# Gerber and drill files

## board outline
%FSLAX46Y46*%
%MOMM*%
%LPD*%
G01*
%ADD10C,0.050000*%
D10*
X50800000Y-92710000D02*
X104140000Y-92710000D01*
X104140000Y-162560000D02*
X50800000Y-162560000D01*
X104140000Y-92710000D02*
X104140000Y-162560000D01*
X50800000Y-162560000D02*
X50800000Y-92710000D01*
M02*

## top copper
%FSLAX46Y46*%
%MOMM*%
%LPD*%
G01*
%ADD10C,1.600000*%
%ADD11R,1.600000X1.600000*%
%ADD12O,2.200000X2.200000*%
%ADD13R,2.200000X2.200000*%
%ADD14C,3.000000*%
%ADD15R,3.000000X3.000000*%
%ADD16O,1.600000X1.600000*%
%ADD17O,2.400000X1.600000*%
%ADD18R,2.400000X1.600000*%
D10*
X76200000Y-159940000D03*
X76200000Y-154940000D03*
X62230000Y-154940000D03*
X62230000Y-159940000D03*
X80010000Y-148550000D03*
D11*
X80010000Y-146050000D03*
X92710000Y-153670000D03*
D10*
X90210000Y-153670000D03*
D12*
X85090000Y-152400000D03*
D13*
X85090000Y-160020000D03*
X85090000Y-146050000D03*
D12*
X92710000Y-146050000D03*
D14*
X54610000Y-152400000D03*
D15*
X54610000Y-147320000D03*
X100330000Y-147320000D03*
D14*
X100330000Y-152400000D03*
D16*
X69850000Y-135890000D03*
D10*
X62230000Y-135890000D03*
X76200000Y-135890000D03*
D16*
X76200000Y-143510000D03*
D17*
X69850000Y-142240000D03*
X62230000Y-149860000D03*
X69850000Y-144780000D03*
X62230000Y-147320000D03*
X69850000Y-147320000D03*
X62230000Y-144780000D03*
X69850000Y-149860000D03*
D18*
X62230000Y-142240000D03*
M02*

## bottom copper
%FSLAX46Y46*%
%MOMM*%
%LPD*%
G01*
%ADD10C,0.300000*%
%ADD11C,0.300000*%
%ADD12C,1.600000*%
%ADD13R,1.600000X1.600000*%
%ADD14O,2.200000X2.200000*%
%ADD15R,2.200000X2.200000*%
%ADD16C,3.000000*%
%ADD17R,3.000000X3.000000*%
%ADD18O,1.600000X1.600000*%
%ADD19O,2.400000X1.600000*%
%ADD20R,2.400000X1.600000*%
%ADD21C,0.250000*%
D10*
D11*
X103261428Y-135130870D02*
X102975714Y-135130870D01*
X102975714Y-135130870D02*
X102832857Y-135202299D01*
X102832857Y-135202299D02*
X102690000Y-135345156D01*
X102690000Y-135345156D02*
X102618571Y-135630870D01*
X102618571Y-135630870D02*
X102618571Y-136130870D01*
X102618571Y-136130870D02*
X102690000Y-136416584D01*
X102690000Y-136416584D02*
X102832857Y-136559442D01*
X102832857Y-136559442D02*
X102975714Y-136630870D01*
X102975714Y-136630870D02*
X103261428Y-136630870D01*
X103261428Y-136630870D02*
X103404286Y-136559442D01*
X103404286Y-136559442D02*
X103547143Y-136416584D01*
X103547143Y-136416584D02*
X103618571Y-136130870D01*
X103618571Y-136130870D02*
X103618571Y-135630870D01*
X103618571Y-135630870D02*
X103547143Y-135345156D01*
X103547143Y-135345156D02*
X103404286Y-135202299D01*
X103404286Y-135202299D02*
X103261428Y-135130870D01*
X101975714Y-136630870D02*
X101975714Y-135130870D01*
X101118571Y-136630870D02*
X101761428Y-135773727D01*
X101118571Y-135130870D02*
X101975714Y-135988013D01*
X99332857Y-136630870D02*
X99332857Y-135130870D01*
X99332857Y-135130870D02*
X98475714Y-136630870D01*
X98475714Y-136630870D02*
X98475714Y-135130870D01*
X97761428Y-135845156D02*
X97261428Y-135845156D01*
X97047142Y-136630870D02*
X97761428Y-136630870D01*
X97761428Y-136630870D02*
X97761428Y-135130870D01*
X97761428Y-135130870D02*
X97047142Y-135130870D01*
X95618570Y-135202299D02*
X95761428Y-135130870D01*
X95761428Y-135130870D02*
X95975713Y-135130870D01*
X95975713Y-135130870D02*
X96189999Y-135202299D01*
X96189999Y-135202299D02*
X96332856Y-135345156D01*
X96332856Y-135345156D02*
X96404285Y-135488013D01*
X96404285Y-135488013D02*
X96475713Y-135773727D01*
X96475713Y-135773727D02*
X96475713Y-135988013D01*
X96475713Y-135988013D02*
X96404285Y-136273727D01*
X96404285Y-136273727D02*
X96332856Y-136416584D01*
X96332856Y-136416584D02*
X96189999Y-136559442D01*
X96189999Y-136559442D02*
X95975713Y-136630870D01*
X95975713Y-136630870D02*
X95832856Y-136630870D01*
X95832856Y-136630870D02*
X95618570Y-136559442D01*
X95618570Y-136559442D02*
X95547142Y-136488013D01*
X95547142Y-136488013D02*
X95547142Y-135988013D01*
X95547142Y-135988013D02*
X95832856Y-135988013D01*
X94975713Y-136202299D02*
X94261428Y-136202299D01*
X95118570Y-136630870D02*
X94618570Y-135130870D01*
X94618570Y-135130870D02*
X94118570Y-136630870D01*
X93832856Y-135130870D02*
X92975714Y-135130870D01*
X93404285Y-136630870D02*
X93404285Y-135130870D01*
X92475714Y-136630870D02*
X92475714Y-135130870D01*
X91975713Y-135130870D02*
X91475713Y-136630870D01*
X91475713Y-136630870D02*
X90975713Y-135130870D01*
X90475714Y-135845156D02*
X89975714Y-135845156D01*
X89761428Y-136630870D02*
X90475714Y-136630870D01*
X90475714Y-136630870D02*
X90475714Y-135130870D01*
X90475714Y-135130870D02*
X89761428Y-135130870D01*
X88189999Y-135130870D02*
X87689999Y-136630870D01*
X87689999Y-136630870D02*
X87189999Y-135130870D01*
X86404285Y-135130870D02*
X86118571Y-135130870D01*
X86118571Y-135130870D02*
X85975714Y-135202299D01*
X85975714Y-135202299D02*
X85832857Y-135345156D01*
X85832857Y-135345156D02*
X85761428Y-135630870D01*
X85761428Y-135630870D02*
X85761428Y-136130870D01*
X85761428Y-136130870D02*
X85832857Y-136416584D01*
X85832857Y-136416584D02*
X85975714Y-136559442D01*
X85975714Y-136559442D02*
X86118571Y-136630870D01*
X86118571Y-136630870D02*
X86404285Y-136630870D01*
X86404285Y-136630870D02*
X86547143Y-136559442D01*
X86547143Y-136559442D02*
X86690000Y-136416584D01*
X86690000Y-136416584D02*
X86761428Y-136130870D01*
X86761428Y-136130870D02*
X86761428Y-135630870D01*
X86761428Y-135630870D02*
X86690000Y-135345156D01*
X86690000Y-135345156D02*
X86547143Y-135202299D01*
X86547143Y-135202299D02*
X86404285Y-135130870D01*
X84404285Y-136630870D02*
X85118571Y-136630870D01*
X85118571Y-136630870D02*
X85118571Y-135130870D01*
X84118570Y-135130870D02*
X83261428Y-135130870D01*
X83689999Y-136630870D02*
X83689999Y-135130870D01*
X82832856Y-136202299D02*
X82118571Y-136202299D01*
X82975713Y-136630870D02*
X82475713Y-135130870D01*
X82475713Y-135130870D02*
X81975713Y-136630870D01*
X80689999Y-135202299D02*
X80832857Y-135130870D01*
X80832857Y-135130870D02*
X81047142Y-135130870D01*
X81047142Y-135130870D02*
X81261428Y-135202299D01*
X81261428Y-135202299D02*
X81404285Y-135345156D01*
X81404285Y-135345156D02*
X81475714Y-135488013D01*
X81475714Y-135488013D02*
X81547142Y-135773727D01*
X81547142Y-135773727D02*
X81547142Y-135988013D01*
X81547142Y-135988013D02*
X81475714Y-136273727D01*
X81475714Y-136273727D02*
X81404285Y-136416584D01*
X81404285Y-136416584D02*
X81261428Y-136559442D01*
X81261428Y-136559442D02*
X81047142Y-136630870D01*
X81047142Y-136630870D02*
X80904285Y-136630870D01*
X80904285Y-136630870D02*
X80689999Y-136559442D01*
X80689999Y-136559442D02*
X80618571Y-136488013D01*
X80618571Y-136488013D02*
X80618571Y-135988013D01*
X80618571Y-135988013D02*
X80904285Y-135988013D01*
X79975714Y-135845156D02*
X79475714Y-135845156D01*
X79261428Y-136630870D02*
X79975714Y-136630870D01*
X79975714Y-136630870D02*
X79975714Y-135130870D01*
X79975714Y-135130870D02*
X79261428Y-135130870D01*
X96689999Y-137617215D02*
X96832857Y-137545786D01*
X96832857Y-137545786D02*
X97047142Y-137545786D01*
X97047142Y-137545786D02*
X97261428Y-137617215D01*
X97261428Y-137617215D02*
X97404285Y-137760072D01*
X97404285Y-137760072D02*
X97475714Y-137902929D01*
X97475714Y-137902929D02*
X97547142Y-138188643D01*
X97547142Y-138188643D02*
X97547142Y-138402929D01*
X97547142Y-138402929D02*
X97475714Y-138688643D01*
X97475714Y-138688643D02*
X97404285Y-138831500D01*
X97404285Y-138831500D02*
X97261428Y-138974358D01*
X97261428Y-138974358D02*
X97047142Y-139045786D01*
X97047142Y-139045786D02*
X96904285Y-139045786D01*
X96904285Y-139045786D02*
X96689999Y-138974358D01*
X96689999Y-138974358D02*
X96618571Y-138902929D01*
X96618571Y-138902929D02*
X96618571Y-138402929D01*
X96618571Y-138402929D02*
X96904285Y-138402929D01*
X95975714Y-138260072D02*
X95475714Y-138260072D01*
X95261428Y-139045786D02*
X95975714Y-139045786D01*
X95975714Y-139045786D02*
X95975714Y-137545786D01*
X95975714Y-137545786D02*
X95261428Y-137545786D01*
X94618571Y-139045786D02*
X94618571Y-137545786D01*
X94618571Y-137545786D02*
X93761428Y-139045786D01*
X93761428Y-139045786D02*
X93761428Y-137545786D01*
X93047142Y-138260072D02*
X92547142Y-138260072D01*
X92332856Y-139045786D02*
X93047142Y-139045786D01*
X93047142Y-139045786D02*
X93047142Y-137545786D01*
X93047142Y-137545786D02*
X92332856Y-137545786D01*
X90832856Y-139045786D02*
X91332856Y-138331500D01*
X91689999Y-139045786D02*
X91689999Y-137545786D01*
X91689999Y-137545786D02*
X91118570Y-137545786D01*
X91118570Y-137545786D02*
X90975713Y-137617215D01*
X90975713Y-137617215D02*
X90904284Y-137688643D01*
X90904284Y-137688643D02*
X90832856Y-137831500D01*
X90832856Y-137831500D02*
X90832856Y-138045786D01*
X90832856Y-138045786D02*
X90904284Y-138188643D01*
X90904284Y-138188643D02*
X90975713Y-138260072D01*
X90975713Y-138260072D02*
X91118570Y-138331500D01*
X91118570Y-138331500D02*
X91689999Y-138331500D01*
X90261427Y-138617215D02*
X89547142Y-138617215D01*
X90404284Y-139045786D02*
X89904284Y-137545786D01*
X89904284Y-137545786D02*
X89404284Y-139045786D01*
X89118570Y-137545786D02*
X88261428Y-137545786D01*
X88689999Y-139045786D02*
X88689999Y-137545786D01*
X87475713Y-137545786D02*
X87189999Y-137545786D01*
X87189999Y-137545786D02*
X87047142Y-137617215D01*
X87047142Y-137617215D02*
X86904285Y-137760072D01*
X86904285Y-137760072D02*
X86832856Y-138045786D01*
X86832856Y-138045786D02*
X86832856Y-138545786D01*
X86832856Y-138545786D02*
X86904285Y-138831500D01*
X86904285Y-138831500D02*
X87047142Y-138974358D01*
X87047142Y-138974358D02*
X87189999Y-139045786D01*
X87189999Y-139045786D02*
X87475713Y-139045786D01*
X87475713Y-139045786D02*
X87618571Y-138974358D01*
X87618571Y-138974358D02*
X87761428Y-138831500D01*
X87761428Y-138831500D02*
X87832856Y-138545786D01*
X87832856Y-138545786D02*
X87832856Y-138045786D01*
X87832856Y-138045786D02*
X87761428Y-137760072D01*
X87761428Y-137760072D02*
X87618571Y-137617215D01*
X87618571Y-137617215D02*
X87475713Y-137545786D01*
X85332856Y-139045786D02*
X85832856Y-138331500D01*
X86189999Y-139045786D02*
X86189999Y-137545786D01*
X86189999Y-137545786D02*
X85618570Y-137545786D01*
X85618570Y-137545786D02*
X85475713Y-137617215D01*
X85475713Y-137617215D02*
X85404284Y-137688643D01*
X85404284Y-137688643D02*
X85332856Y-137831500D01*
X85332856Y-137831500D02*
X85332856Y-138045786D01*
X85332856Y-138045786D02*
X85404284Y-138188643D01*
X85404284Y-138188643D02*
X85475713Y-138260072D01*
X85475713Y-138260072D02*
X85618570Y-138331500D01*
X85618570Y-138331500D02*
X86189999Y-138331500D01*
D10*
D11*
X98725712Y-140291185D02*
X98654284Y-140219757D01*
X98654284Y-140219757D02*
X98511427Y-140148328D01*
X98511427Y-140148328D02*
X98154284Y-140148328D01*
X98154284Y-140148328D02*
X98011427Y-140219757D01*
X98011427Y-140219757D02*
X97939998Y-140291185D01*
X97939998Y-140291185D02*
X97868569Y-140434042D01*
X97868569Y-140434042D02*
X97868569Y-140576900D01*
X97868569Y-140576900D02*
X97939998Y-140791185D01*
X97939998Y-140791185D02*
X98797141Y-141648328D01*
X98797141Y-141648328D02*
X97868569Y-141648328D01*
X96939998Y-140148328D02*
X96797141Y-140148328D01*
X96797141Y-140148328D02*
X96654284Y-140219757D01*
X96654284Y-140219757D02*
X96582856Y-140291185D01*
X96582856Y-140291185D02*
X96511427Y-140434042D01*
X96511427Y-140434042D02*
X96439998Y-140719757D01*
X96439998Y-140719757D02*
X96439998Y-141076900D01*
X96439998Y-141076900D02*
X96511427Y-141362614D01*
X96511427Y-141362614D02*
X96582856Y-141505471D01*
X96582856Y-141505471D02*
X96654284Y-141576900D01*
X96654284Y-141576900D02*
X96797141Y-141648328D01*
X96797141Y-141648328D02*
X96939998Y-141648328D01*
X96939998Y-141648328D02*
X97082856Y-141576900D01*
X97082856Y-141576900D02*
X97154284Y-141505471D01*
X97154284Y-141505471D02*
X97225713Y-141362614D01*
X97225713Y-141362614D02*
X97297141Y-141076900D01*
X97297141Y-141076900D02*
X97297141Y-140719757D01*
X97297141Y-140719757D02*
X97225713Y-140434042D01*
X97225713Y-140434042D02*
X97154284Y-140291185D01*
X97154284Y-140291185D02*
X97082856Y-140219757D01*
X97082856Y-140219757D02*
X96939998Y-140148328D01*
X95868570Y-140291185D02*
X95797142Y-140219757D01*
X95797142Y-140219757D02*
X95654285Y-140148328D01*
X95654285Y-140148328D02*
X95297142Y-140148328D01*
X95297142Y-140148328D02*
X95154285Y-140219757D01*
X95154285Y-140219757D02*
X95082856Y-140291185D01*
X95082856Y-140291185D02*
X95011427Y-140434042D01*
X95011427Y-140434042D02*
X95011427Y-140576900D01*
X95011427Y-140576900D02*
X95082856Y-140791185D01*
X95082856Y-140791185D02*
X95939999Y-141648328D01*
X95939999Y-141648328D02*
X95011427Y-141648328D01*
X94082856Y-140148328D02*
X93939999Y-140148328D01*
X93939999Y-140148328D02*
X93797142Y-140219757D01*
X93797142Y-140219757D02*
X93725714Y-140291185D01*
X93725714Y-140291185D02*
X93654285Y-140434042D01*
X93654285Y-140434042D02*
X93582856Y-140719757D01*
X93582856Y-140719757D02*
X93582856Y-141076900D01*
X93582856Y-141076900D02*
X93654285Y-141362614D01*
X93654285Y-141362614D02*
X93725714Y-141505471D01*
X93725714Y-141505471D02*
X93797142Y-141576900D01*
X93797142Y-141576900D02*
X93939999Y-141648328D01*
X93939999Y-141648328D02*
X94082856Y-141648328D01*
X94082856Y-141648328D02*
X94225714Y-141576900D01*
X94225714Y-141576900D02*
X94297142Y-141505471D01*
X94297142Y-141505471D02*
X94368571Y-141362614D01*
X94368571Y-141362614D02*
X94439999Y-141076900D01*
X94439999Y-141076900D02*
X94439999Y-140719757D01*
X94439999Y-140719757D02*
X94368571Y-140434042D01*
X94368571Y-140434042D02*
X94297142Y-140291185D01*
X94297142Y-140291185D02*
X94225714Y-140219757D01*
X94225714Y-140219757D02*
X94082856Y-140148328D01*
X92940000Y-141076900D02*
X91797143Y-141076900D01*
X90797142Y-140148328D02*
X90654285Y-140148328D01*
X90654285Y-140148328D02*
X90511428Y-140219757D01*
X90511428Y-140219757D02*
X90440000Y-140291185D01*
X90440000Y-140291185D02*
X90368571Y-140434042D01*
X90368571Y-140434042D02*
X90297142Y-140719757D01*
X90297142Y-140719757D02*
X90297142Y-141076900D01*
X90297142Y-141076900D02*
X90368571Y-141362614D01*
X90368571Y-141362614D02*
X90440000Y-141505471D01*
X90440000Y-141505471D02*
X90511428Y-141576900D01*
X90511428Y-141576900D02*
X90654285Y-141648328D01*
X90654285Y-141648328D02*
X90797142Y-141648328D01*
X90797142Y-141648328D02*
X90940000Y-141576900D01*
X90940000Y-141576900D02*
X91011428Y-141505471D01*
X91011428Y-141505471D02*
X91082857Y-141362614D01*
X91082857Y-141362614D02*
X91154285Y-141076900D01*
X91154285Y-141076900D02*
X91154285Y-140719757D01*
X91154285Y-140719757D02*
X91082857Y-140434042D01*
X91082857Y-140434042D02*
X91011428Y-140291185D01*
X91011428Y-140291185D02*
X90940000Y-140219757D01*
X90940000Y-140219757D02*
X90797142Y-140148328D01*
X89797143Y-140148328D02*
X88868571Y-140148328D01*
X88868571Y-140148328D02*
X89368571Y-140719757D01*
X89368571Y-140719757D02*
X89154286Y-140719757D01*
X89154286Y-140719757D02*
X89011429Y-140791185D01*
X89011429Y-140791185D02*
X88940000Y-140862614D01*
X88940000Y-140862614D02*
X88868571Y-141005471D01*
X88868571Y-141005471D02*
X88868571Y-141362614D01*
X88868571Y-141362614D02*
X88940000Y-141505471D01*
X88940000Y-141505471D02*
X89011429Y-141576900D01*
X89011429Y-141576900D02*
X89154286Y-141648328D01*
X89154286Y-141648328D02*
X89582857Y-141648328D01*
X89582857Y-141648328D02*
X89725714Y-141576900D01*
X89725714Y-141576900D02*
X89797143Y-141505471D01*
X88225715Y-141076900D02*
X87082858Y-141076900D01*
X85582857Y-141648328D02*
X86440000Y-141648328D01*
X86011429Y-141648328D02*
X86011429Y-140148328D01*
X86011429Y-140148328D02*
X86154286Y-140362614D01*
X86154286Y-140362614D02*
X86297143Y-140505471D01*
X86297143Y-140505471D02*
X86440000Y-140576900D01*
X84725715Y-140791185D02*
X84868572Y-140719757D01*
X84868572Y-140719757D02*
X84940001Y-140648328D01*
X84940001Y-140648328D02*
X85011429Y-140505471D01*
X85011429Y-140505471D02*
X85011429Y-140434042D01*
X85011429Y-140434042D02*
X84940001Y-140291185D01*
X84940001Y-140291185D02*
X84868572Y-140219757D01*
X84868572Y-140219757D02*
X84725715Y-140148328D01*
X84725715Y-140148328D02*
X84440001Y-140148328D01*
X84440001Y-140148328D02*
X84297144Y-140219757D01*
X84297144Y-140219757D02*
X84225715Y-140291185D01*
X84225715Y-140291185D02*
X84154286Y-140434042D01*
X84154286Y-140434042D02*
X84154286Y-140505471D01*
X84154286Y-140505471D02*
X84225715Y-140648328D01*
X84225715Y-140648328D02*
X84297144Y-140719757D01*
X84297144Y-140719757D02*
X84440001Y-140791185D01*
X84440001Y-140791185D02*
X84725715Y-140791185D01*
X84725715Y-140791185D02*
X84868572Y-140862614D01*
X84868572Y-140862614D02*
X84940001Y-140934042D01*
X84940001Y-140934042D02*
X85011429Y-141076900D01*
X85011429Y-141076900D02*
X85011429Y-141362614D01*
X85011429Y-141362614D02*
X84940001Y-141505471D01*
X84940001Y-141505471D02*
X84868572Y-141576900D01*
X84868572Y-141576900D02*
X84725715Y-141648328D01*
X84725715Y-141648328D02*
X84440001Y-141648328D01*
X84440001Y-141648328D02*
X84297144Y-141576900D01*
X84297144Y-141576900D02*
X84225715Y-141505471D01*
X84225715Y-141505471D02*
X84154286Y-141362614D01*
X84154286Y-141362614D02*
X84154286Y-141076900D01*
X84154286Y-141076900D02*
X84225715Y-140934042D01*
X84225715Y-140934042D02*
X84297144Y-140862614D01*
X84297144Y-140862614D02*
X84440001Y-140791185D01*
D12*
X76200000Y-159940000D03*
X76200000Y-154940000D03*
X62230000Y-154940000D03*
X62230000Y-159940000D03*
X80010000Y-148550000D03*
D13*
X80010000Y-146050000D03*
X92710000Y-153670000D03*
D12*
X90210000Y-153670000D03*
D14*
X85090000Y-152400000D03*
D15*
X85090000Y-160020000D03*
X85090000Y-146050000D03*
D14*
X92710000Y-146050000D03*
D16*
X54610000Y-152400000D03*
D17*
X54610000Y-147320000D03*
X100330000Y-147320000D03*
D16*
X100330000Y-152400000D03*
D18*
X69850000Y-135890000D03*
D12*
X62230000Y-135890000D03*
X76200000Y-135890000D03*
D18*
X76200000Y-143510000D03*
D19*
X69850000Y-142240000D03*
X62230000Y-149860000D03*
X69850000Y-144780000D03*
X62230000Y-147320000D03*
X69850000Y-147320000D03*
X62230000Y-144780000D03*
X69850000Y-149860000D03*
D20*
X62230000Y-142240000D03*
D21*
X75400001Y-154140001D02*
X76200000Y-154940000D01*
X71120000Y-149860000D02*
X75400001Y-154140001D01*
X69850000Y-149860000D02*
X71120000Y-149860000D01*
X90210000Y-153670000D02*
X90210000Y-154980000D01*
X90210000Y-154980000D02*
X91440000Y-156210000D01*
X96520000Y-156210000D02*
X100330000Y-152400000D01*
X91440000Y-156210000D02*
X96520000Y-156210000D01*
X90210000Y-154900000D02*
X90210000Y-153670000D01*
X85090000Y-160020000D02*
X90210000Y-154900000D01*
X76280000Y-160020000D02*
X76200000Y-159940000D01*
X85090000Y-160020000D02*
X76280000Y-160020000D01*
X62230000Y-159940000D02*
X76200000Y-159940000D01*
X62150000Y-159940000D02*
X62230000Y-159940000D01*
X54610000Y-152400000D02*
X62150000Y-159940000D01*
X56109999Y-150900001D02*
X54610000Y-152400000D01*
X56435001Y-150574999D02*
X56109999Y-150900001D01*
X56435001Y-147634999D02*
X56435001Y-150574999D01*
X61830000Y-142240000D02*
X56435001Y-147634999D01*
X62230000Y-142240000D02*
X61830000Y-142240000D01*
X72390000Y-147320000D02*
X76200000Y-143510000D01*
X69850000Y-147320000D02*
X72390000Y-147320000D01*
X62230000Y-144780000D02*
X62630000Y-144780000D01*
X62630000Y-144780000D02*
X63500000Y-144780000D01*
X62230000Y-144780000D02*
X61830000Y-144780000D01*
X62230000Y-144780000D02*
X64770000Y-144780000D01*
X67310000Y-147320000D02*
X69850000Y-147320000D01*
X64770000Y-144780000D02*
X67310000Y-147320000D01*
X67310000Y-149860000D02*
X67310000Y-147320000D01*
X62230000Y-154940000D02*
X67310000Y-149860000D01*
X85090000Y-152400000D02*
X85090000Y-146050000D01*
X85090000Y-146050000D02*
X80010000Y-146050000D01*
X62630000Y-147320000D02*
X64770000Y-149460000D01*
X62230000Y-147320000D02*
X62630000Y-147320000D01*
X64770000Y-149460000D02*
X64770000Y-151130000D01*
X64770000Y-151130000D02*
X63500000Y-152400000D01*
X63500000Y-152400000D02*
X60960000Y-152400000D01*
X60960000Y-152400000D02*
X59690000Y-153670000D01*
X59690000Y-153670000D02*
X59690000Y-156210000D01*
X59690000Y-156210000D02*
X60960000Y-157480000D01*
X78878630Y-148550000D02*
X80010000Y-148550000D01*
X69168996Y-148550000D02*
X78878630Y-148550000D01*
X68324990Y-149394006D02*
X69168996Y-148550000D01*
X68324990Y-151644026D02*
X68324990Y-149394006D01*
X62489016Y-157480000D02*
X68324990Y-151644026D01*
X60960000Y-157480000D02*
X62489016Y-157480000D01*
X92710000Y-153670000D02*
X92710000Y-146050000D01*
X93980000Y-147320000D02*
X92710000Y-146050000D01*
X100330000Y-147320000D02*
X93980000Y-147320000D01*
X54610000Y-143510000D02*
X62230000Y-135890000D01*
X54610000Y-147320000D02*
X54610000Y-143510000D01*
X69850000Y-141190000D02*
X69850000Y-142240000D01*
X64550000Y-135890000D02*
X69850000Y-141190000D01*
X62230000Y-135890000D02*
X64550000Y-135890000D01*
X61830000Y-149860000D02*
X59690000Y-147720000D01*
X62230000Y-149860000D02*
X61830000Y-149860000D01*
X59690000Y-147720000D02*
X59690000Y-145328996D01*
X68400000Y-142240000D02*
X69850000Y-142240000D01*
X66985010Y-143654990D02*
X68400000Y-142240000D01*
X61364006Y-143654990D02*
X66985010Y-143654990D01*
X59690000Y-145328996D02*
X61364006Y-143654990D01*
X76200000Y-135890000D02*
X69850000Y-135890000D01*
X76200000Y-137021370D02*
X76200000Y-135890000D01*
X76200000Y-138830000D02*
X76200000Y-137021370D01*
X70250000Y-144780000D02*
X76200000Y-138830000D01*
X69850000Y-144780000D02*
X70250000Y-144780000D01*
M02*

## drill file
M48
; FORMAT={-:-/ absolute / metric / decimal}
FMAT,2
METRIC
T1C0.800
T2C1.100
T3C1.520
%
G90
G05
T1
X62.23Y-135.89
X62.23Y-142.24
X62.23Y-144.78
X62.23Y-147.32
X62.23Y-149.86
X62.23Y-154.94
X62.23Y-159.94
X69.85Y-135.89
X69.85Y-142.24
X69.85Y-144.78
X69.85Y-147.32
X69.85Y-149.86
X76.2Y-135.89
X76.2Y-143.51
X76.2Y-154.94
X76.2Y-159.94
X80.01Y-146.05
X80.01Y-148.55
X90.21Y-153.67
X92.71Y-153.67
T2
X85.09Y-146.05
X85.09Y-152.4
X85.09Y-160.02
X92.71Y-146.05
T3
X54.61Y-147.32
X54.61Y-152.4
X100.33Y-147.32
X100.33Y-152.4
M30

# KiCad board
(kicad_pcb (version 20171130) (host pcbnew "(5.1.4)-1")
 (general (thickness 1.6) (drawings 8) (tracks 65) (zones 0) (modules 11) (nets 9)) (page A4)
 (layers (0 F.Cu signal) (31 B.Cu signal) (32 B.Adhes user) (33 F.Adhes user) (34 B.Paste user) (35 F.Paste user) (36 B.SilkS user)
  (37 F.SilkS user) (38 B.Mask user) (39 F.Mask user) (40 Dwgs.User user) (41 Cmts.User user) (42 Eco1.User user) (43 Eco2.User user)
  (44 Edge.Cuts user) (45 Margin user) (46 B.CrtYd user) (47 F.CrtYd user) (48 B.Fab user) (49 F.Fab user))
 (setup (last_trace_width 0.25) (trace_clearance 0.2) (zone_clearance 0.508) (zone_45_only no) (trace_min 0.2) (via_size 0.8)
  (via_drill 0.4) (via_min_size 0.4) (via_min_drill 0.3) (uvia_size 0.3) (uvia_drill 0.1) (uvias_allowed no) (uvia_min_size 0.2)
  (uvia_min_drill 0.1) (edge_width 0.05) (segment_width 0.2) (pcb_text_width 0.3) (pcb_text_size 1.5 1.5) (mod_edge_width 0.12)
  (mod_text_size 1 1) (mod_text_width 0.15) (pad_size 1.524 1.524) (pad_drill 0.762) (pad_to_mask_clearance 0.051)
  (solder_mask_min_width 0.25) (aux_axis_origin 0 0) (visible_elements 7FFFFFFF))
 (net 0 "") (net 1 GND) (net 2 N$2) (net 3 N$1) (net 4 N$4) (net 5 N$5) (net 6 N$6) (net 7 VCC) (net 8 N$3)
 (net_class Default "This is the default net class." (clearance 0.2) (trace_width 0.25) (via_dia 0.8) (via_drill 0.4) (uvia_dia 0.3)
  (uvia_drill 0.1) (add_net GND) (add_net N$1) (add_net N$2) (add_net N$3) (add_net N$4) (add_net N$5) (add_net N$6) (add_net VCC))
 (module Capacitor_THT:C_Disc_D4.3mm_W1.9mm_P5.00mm (layer F.Cu) (at 76.2 154.94 270)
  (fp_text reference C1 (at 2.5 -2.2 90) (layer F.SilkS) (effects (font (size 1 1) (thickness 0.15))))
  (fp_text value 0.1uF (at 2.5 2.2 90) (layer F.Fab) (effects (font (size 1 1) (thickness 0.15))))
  (pad 2 thru_hole circle (at 5 0 270) (size 1.6 1.6) (drill 0.8) (layers *.Cu *.Mask) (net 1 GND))
  (pad 1 thru_hole circle (at 0 0 270) (size 1.6 1.6) (drill 0.8) (layers *.Cu *.Mask) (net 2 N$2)))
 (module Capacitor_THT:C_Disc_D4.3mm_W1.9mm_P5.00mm (layer F.Cu) (at 62.23 154.94 270)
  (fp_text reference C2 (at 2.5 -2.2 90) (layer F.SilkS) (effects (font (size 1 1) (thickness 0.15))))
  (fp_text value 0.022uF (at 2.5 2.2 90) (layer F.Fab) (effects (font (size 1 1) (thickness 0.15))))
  (pad 1 thru_hole circle (at 0 0 270) (size 1.6 1.6) (drill 0.8) (layers *.Cu *.Mask) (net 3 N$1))
  (pad 2 thru_hole circle (at 5 0 270) (size 1.6 1.6) (drill 0.8) (layers *.Cu *.Mask) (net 1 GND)))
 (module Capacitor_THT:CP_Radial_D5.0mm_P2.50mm (layer F.Cu) (at 80.01 146.05 270)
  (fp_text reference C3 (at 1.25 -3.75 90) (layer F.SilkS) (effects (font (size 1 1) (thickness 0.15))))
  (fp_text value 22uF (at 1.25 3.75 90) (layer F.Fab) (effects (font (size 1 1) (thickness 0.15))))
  (pad 2 thru_hole circle (at 2.5 0 270) (size 1.6 1.6) (drill 0.8) (layers *.Cu *.Mask) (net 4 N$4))
  (pad 1 thru_hole rect (at 0 0 270) (size 1.6 1.6) (drill 0.8) (layers *.Cu *.Mask) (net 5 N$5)))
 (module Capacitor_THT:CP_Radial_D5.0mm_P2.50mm (layer F.Cu) (at 92.71 153.67 180)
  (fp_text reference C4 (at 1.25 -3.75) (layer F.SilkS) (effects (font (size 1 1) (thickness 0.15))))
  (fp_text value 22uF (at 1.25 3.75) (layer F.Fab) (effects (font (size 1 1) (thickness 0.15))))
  (pad 1 thru_hole rect (at 0 0 180) (size 1.6 1.6) (drill 0.8) (layers *.Cu *.Mask) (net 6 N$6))
  (pad 2 thru_hole circle (at 2.5 0 180) (size 1.6 1.6) (drill 0.8) (layers *.Cu *.Mask) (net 1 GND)))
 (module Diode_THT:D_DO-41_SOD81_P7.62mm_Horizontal (layer F.Cu) (at 85.09 160.02 90)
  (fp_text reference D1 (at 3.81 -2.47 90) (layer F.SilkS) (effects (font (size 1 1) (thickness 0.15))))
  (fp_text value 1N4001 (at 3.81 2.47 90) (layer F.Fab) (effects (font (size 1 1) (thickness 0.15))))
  (pad 2 thru_hole oval (at 7.62 0 90) (size 2.2 2.2) (drill 1.1) (layers *.Cu *.Mask) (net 5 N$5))
  (pad 1 thru_hole rect (at 0 0 90) (size 2.2 2.2) (drill 1.1) (layers *.Cu *.Mask) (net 1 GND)))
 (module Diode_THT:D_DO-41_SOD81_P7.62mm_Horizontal (layer F.Cu) (at 85.09 146.05)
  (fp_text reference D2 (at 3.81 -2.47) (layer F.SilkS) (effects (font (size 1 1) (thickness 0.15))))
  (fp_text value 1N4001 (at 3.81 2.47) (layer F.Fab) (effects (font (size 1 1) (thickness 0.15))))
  (pad 1 thru_hole rect (at 0 0) (size 2.2 2.2) (drill 1.1) (layers *.Cu *.Mask) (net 5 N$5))
  (pad 2 thru_hole oval (at 7.62 0) (size 2.2 2.2) (drill 1.1) (layers *.Cu *.Mask) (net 6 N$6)))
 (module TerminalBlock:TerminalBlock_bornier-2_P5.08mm (layer F.Cu) (at 54.61 147.32 270)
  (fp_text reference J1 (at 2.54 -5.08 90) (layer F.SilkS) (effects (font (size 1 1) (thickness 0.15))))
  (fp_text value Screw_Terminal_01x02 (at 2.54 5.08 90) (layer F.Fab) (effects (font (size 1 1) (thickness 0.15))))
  (pad 2 thru_hole circle (at 5.08 0 270) (size 3 3) (drill 1.52) (layers *.Cu *.Mask) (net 1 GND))
  (pad 1 thru_hole rect (at 0 0 270) (size 3 3) (drill 1.52) (layers *.Cu *.Mask) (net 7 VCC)))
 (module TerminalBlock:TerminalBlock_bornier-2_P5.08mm (layer F.Cu) (at 100.33 147.32 270)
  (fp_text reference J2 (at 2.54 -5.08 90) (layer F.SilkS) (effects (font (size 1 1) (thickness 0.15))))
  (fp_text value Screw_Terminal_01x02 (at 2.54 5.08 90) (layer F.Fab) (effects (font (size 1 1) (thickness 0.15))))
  (pad 1 thru_hole rect (at 0 0 270) (size 3 3) (drill 1.52) (layers *.Cu *.Mask) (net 6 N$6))
  (pad 2 thru_hole circle (at 5.08 0 270) (size 3 3) (drill 1.52) (layers *.Cu *.Mask) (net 1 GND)))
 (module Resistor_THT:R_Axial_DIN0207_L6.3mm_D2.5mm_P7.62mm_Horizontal (layer F.Cu) (at 62.23 135.89)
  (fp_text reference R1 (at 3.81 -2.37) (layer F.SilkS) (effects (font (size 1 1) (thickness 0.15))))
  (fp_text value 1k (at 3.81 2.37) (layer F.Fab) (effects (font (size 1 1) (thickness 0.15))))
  (pad 2 thru_hole oval (at 7.62 0) (size 1.6 1.6) (drill 0.8) (layers *.Cu *.Mask) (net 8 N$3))
  (pad 1 thru_hole circle (at 0 0) (size 1.6 1.6) (drill 0.8) (layers *.Cu *.Mask) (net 7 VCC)))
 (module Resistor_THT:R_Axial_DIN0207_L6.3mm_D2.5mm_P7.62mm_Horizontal (layer F.Cu) (at 76.2 135.89 270)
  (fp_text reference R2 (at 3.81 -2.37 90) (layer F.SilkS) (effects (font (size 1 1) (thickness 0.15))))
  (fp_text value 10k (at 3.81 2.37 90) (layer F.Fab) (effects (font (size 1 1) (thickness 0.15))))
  (pad 1 thru_hole circle (at 0 0 270) (size 1.6 1.6) (drill 0.8) (layers *.Cu *.Mask) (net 8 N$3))
  (pad 2 thru_hole oval (at 7.62 0 270) (size 1.6 1.6) (drill 0.8) (layers *.Cu *.Mask) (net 3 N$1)))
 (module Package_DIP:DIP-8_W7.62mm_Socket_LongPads (layer F.Cu) (at 62.23 142.24)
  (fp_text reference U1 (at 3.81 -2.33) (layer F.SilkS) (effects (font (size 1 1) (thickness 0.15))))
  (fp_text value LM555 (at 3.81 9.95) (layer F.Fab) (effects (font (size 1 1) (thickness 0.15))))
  (pad 8 thru_hole oval (at 7.62 0) (size 2.4 1.6) (drill 0.8) (layers *.Cu *.Mask) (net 7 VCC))
  (pad 4 thru_hole oval (at 0 7.62) (size 2.4 1.6) (drill 0.8) (layers *.Cu *.Mask) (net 7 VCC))
  (pad 7 thru_hole oval (at 7.62 2.54) (size 2.4 1.6) (drill 0.8) (layers *.Cu *.Mask) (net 8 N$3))
  (pad 3 thru_hole oval (at 0 5.08) (size 2.4 1.6) (drill 0.8) (layers *.Cu *.Mask) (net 4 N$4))
  (pad 6 thru_hole oval (at 7.62 5.08) (size 2.4 1.6) (drill 0.8) (layers *.Cu *.Mask) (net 3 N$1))
  (pad 2 thru_hole oval (at 0 2.54) (size 2.4 1.6) (drill 0.8) (layers *.Cu *.Mask) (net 3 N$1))
  (pad 5 thru_hole oval (at 7.62 7.62) (size 2.4 1.6) (drill 0.8) (layers *.Cu *.Mask) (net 2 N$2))
  (pad 1 thru_hole rect (at 0 0) (size 2.4 1.6) (drill 0.8) (layers *.Cu *.Mask) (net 1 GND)))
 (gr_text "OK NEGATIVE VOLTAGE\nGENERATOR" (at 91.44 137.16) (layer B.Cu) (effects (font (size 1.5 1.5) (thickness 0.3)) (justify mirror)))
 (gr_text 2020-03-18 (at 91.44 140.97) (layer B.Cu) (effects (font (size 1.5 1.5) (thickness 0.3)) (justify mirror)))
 (gr_line (start 50.8 92.71) (end 104.14 92.71) (layer Edge.Cuts) (width 0.05))
 (gr_line (start 104.14 162.56) (end 50.8 162.56) (layer Edge.Cuts) (width 0.05))
 (gr_line (start 104.14 92.71) (end 104.14 162.56) (layer Edge.Cuts) (width 0.05))
 (gr_line (start 50.8 162.56) (end 50.8 92.71) (layer Edge.Cuts) (width 0.05))
 (segment (start 75.400001 154.140001) (end 76.2 154.94) (width 0.25) (layer B.Cu) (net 2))
 (segment (start 71.12 149.86) (end 75.400001 154.140001) (width 0.25) (layer B.Cu) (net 2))
 (segment (start 69.85 149.86) (end 71.12 149.86) (width 0.25) (layer B.Cu) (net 2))
 (segment (start 90.21 153.67) (end 90.21 154.98) (width 0.25) (layer B.Cu) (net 1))
 (segment (start 90.21 154.98) (end 91.44 156.21) (width 0.25) (layer B.Cu) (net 1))
 (segment (start 96.52 156.21) (end 100.33 152.4) (width 0.25) (layer B.Cu) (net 1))
 (segment (start 91.44 156.21) (end 96.52 156.21) (width 0.25) (layer B.Cu) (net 1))
 (segment (start 90.21 154.9) (end 90.21 153.67) (width 0.25) (layer B.Cu) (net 1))
 (segment (start 85.09 160.02) (end 90.21 154.9) (width 0.25) (layer B.Cu) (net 1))
 (segment (start 76.28 160.02) (end 76.2 159.94) (width 0.25) (layer B.Cu) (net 1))
 (segment (start 85.09 160.02) (end 76.28 160.02) (width 0.25) (layer B.Cu) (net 1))
 (segment (start 62.23 159.94) (end 76.2 159.94) (width 0.25) (layer B.Cu) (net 1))
 (segment (start 62.15 159.94) (end 62.23 159.94) (width 0.25) (layer B.Cu) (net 1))
 (segment (start 54.61 152.4) (end 62.15 159.94) (width 0.25) (layer B.Cu) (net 1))
 (segment (start 56.109999 150.900001) (end 54.61 152.4) (width 0.25) (layer B.Cu) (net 1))
 (segment (start 56.435001 150.574999) (end 56.109999 150.900001) (width 0.25) (layer B.Cu) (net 1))
 (segment (start 56.435001 147.634999) (end 56.435001 150.574999) (width 0.25) (layer B.Cu) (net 1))
 (segment (start 61.83 142.24) (end 56.435001 147.634999) (width 0.25) (layer B.Cu) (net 1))
 (segment (start 62.23 142.24) (end 61.83 142.24) (width 0.25) (layer B.Cu) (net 1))
 (segment (start 72.39 147.32) (end 76.2 143.51) (width 0.25) (layer B.Cu) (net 3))
 (segment (start 69.85 147.32) (end 72.39 147.32) (width 0.25) (layer B.Cu) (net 3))
 (segment (start 62.23 144.78) (end 62.63 144.78) (width 0.25) (layer B.Cu) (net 3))
 (segment (start 62.63 144.78) (end 63.5 144.78) (width 0.25) (layer B.Cu) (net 3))
 (segment (start 62.23 144.78) (end 61.83 144.78) (width 0.25) (layer B.Cu) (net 3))
 (segment (start 62.23 144.78) (end 64.77 144.78) (width 0.25) (layer B.Cu) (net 3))
 (segment (start 67.31 147.32) (end 69.85 147.32) (width 0.25) (layer B.Cu) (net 3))
 (segment (start 64.77 144.78) (end 67.31 147.32) (width 0.25) (layer B.Cu) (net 3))
 (segment (start 67.31 149.86) (end 67.31 147.32) (width 0.25) (layer B.Cu) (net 3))
 (segment (start 62.23 154.94) (end 67.31 149.86) (width 0.25) (layer B.Cu) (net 3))
 (segment (start 85.09 152.4) (end 85.09 146.05) (width 0.25) (layer B.Cu) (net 5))
 (segment (start 85.09 146.05) (end 80.01 146.05) (width 0.25) (layer B.Cu) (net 5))
 (segment (start 62.63 147.32) (end 64.77 149.46) (width 0.25) (layer B.Cu) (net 4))
 (segment (start 62.23 147.32) (end 62.63 147.32) (width 0.25) (layer B.Cu) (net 4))
 (segment (start 64.77 149.46) (end 64.77 151.13) (width 0.25) (layer B.Cu) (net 4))
 (segment (start 64.77 151.13) (end 63.5 152.4) (width 0.25) (layer B.Cu) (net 4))
 (segment (start 63.5 152.4) (end 60.96 152.4) (width 0.25) (layer B.Cu) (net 4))
 (segment (start 60.96 152.4) (end 59.69 153.67) (width 0.25) (layer B.Cu) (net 4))
 (segment (start 59.69 153.67) (end 59.69 156.21) (width 0.25) (layer B.Cu) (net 4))
 (segment (start 59.69 156.21) (end 60.96 157.48) (width 0.25) (layer B.Cu) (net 4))
 (segment (start 78.87863 148.55) (end 80.01 148.55) (width 0.25) (layer B.Cu) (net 4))
 (segment (start 69.168996 148.55) (end 78.87863 148.55) (width 0.25) (layer B.Cu) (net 4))
 (segment (start 68.32499 149.394006) (end 69.168996 148.55) (width 0.25) (layer B.Cu) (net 4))
 (segment (start 68.32499 151.644026) (end 68.32499 149.394006) (width 0.25) (layer B.Cu) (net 4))
 (segment (start 62.489016 157.48) (end 68.32499 151.644026) (width 0.25) (layer B.Cu) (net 4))
 (segment (start 60.96 157.48) (end 62.489016 157.48) (width 0.25) (layer B.Cu) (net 4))
 (segment (start 92.71 153.67) (end 92.71 146.05) (width 0.25) (layer B.Cu) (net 6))
 (segment (start 93.98 147.32) (end 92.71 146.05) (width 0.25) (layer B.Cu) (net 6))
 (segment (start 100.33 147.32) (end 93.98 147.32) (width 0.25) (layer B.Cu) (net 6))
 (segment (start 54.61 143.51) (end 62.23 135.89) (width 0.25) (layer B.Cu) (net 7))
 (segment (start 54.61 147.32) (end 54.61 143.51) (width 0.25) (layer B.Cu) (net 7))
 (segment (start 69.85 141.19) (end 69.85 142.24) (width 0.25) (layer B.Cu) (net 7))
 (segment (start 64.55 135.89) (end 69.85 141.19) (width 0.25) (layer B.Cu) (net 7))
 (segment (start 62.23 135.89) (end 64.55 135.89) (width 0.25) (layer B.Cu) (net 7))
 (segment (start 61.83 149.86) (end 59.69 147.72) (width 0.25) (layer B.Cu) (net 7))
 (segment (start 62.23 149.86) (end 61.83 149.86) (width 0.25) (layer B.Cu) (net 7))
 (segment (start 59.69 147.72) (end 59.69 145.328996) (width 0.25) (layer B.Cu) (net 7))
 (segment (start 68.4 142.24) (end 69.85 142.24) (width 0.25) (layer B.Cu) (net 7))
 (segment (start 66.98501 143.65499) (end 68.4 142.24) (width 0.25) (layer B.Cu) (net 7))
 (segment (start 61.364006 143.65499) (end 66.98501 143.65499) (width 0.25) (layer B.Cu) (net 7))
 (segment (start 59.69 145.328996) (end 61.364006 143.65499) (width 0.25) (layer B.Cu) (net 7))
 (segment (start 76.2 135.89) (end 69.85 135.89) (width 0.25) (layer B.Cu) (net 8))
 (segment (start 76.2 137.02137) (end 76.2 135.89) (width 0.25) (layer B.Cu) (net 8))
 (segment (start 76.2 138.83) (end 76.2 137.02137) (width 0.25) (layer B.Cu) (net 8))
 (segment (start 70.25 144.78) (end 76.2 138.83) (width 0.25) (layer B.Cu) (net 8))
 (segment (start 69.85 144.78) (end 70.25 144.78) (width 0.25) (layer B.Cu) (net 8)))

